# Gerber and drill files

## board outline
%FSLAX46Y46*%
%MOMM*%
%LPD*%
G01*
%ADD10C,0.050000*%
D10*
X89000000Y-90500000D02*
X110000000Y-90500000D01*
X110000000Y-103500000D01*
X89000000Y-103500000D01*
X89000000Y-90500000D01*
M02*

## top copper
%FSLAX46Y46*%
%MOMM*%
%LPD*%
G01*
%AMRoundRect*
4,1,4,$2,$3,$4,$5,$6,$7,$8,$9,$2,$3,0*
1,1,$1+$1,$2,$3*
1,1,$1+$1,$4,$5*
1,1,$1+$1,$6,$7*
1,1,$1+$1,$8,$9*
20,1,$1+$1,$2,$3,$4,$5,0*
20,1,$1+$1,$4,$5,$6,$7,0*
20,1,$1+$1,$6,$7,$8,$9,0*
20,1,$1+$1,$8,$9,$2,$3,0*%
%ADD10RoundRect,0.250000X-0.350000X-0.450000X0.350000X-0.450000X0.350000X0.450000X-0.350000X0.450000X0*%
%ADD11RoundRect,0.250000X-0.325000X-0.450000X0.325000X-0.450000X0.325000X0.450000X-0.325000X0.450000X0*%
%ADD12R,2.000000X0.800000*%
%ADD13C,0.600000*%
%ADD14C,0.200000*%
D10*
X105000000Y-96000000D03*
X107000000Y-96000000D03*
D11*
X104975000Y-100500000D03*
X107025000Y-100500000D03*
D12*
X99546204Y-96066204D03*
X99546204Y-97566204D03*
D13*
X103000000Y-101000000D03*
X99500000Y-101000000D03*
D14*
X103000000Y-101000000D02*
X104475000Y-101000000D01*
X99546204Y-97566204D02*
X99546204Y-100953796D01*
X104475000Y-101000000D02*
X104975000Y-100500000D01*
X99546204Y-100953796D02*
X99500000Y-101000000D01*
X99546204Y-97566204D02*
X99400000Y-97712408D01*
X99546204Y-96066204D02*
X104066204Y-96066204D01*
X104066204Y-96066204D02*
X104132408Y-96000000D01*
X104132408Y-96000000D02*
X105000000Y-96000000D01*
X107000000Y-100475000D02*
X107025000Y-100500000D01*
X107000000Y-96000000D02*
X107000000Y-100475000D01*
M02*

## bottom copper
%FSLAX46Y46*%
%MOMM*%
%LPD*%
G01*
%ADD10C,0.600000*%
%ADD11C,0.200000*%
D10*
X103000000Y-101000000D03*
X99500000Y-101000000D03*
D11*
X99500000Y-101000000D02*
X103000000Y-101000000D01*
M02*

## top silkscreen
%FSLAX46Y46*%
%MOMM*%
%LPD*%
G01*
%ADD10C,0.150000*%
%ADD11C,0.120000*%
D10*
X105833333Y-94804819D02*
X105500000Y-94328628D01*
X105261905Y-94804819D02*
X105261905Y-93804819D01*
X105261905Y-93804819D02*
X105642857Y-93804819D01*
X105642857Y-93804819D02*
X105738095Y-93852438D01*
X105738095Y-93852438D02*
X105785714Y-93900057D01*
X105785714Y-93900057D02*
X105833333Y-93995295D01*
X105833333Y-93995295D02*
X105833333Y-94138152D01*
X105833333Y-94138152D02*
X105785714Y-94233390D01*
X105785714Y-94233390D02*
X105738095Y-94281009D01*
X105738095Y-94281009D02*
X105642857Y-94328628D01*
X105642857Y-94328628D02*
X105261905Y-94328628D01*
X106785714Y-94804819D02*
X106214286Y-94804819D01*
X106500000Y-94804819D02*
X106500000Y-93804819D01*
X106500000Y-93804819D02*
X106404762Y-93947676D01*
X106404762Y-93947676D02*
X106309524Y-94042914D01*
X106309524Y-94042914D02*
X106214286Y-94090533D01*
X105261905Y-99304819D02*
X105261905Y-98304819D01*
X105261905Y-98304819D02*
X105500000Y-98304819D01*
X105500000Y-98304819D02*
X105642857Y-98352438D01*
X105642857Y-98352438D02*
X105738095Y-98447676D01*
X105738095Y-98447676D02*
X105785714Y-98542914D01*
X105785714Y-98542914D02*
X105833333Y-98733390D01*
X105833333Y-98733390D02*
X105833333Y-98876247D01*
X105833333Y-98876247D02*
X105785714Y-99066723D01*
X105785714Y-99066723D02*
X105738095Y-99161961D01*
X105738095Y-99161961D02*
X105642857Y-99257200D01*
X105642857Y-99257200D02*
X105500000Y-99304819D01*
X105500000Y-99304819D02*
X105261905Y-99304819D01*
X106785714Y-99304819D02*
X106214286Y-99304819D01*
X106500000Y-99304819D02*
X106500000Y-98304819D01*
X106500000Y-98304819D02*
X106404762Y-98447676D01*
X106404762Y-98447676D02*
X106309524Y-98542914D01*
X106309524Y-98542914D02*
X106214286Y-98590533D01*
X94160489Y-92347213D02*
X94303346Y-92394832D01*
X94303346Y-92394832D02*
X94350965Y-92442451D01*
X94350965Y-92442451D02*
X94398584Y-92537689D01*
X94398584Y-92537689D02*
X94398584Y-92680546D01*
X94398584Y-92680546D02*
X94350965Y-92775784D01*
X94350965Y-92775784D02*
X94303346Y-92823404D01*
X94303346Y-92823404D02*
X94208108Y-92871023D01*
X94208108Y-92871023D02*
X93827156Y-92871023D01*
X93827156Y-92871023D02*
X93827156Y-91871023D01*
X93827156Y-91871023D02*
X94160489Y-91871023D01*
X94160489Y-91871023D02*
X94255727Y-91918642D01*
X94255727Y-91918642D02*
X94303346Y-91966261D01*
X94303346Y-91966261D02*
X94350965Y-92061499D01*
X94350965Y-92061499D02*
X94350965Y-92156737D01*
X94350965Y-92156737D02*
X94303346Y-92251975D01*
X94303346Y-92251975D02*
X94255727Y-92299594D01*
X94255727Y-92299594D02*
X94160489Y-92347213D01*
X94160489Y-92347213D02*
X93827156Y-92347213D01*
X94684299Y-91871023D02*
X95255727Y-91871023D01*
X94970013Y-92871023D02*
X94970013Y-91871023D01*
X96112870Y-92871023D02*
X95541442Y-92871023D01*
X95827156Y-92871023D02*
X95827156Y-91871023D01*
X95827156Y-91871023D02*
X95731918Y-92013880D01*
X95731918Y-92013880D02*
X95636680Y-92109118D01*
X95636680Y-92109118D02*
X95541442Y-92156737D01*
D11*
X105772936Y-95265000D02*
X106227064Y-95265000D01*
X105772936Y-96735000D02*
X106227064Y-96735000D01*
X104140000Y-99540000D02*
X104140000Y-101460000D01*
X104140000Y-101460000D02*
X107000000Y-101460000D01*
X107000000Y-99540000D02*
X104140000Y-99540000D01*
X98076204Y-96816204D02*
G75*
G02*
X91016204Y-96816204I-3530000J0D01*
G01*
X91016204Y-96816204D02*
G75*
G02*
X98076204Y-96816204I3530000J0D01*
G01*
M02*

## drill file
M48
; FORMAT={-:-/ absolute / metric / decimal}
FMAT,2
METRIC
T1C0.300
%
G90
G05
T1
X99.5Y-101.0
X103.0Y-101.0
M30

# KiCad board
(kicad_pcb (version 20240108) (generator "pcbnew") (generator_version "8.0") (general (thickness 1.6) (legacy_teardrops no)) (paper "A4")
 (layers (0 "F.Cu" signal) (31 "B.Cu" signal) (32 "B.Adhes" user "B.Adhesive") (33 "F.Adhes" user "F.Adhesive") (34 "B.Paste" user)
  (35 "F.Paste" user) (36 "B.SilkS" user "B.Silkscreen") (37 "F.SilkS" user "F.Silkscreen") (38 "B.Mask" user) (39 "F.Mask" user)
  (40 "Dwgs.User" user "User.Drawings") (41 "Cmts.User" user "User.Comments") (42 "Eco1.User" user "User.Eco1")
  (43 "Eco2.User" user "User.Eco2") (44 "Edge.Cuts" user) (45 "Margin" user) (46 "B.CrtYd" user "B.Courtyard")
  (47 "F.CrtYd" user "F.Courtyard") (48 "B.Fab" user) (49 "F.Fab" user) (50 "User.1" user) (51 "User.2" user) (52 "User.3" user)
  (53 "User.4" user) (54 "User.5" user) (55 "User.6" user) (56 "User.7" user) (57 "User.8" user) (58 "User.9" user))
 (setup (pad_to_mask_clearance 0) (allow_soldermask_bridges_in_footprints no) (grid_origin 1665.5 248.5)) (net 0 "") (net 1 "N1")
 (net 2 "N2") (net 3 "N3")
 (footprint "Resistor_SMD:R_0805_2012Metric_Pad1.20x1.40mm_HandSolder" (layer "F.Cu") (at 106 96)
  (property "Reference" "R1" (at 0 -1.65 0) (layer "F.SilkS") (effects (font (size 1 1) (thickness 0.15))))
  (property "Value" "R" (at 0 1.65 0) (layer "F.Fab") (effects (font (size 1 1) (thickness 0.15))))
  (fp_line (start -0.227064 -0.735) (end 0.227064 -0.735) (stroke (width 0.12) (type solid)) (layer "F.SilkS"))
  (fp_line (start -0.227064 0.735) (end 0.227064 0.735) (stroke (width 0.12) (type solid)) (layer "F.SilkS"))
  (pad "1" smd roundrect (at -1 0) (size 1.2 1.4) (layers "F.Cu" "F.Paste" "F.Mask") (roundrect_rratio 0.208333) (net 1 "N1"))
  (pad "2" smd roundrect (at 1 0) (size 1.2 1.4) (layers "F.Cu" "F.Paste" "F.Mask") (roundrect_rratio 0.208333) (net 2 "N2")))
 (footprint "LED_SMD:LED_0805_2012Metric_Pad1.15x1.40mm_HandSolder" (layer "F.Cu") (at 106 100.5)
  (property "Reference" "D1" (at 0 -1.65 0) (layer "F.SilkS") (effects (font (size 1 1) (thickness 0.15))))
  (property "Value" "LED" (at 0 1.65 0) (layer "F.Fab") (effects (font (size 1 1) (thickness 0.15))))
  (fp_line (start -1.86 -0.96) (end -1.86 0.96) (stroke (width 0.12) (type solid)) (layer "F.SilkS"))
  (fp_line (start -1.86 0.96) (end 1 0.96) (stroke (width 0.12) (type solid)) (layer "F.SilkS"))
  (fp_line (start 1 -0.96) (end -1.86 -0.96) (stroke (width 0.12) (type solid)) (layer "F.SilkS"))
  (pad "1" smd roundrect (at -1.025 0) (size 1.15 1.4) (layers "F.Cu" "F.Paste" "F.Mask") (roundrect_rratio 0.217391) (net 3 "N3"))
  (pad "2" smd roundrect (at 1.025 0) (size 1.15 1.4) (layers "F.Cu" "F.Paste" "F.Mask") (roundrect_rratio 0.217391) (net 2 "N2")))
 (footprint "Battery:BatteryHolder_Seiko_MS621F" (layer "F.Cu") (at 99.546204 96.816204)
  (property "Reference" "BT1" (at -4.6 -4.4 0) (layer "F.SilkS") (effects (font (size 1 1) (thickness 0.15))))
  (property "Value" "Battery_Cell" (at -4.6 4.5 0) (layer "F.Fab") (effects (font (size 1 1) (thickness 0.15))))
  (fp_circle (center -5 0) (end -1.47 0) (stroke (width 0.12) (type solid)) (fill none) (layer "F.SilkS"))
  (pad "1" smd rect (at 0 -0.75) (size 2 0.8) (layers "F.Cu" "F.Paste" "F.Mask") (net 1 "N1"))
  (pad "2" smd rect (at 0 0.75) (size 2 0.8) (layers "F.Cu" "F.Paste" "F.Mask") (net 3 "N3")))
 (gr_rect (start 89 90.5) (end 110 103.5) (stroke (width 0.05) (type default)) (fill none) (layer "Edge.Cuts"))
 (segment (start 103 101) (end 104.475 101) (width 0.2) (layer "F.Cu") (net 3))
 (segment (start 99.546204 97.566204) (end 99.546204 100.953796) (width 0.2) (layer "F.Cu") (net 3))
 (segment (start 104.475 101) (end 104.975 100.5) (width 0.2) (layer "F.Cu") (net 3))
 (segment (start 99.546204 100.953796) (end 99.5 101) (width 0.2) (layer "F.Cu") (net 3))
 (segment (start 99.546204 97.566204) (end 99.4 97.712408) (width 0.2) (layer "F.Cu") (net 3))
 (via (at 103 101) (size 0.6) (drill 0.3) (layers "F.Cu" "B.Cu") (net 3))
 (via (at 99.5 101) (size 0.6) (drill 0.3) (layers "F.Cu" "B.Cu") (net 3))
 (segment (start 99.5 101) (end 103 101) (width 0.2) (layer "B.Cu") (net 3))
 (segment (start 99.546204 96.066204) (end 104.066204 96.066204) (width 0.2) (layer "F.Cu") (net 1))
 (segment (start 104.066204 96.066204) (end 104.132408 96) (width 0.2) (layer "F.Cu") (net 1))
 (segment (start 104.132408 96) (end 105 96) (width 0.2) (layer "F.Cu") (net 1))
 (segment (start 107 100.475) (end 107.025 100.5) (width 0.2) (layer "F.Cu") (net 2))
 (segment (start 107 96) (end 107 100.475) (width 0.2) (layer "F.Cu") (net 2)))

